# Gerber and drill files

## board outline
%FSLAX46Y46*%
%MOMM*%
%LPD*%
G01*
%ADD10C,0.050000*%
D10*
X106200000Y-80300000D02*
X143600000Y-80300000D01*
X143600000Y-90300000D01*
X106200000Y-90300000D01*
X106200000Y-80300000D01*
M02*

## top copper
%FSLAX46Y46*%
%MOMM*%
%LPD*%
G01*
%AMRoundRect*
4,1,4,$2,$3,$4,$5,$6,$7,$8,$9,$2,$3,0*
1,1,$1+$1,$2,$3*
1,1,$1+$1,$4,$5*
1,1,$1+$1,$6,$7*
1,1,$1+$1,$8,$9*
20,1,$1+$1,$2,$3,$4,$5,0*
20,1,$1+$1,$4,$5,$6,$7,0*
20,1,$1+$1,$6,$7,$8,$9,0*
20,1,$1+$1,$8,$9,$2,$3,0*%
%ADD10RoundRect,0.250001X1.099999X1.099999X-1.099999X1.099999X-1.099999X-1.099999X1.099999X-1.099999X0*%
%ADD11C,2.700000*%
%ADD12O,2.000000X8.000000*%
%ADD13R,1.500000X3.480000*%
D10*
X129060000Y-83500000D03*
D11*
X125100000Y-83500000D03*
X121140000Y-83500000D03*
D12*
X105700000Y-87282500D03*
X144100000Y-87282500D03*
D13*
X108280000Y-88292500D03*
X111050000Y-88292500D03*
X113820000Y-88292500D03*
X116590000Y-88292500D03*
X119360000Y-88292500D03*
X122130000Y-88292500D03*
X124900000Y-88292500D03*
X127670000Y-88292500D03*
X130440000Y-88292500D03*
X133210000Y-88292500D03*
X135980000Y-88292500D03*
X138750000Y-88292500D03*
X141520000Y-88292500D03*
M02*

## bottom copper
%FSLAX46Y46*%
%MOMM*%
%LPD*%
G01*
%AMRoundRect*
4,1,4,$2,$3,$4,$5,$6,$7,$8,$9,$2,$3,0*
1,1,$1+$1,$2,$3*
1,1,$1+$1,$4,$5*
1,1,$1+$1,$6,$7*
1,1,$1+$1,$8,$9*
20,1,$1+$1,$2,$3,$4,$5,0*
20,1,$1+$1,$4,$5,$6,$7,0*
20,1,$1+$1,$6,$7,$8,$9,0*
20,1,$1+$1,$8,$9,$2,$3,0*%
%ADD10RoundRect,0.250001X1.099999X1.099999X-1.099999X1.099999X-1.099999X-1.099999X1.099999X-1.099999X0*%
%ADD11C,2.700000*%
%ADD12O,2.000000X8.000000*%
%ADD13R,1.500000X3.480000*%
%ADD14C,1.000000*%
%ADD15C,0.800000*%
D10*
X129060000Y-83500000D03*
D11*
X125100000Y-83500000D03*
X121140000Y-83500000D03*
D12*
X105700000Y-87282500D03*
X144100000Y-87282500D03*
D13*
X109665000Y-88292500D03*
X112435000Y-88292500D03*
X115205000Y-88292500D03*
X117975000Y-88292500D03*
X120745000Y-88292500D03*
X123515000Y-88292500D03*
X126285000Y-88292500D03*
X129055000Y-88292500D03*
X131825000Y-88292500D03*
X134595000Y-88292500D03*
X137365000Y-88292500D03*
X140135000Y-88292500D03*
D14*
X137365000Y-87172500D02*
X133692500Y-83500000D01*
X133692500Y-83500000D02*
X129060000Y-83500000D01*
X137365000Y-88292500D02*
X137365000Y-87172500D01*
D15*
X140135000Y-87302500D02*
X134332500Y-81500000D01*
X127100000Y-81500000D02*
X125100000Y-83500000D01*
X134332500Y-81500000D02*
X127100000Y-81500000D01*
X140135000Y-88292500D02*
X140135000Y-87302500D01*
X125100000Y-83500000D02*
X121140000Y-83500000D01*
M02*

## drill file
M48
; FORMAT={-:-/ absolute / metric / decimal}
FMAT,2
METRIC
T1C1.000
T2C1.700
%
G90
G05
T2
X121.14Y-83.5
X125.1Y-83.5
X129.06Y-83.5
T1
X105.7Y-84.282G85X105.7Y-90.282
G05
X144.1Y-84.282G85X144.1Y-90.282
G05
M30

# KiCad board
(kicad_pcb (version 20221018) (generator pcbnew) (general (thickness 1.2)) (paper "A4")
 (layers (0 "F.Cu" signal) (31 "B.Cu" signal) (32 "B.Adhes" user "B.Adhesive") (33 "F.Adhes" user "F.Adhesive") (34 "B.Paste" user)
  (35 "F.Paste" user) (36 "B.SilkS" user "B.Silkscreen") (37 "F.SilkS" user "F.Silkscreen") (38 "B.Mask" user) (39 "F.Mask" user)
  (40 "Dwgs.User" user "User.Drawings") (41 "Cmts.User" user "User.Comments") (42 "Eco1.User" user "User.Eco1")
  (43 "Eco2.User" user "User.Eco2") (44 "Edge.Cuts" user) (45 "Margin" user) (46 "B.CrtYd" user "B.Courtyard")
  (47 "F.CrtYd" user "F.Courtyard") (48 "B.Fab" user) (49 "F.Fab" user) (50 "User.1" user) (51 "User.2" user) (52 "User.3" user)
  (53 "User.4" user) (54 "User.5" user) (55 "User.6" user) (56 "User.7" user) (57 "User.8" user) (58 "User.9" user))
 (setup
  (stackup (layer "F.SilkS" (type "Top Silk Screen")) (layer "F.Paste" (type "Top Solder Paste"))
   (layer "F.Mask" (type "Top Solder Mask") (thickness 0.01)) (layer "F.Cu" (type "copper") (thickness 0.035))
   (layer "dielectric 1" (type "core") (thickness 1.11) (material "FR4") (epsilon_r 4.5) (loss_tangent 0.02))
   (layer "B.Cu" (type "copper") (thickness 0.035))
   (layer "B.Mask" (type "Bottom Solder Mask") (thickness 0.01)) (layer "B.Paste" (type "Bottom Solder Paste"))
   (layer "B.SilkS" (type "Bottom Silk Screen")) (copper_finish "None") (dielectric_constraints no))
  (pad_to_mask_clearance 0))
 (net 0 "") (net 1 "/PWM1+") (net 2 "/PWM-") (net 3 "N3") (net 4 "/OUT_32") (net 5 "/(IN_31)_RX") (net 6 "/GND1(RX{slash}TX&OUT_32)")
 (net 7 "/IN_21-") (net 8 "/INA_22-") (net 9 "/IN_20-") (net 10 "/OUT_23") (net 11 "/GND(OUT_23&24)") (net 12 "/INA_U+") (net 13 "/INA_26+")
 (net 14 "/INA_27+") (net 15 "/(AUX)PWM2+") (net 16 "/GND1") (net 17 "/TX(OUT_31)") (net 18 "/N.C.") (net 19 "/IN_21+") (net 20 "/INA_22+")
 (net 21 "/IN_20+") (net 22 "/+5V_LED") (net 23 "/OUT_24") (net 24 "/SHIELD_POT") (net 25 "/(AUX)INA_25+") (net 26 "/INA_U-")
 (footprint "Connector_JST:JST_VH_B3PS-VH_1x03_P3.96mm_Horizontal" (layer "F.Cu") (at 129.06 83.5 180)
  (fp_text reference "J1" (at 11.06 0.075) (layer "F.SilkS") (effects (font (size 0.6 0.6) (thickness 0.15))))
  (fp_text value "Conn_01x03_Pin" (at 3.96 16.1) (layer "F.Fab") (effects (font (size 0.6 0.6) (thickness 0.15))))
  (pad "1" thru_hole roundrect (at 0 0 180) (size 2.7 2.7) (drill 1.7) (layers "*.Cu" "*.Mask") (roundrect_rratio 0.092593) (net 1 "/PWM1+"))
  (pad "2" thru_hole circle (at 3.96 0 180) (size 2.7 2.7) (drill 1.7) (layers "*.Cu" "*.Mask") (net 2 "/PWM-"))
  (pad "3" thru_hole circle (at 7.92 0 180) (size 2.7 2.7) (drill 1.7) (layers "*.Cu" "*.Mask") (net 2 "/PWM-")))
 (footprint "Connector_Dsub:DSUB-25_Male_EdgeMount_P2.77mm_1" (layer "F.Cu") (at 124.9 88.2925)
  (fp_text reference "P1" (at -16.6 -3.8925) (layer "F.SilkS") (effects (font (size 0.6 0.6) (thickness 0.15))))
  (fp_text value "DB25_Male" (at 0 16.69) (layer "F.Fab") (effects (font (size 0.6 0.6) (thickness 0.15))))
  (pad "0" thru_hole oval (at -19.2 -1.01) (size 2 8) (drill oval 1 7) (layers "*.Cu" "*.Mask") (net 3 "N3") (thermal_bridge_angle 45))
  (pad "0" thru_hole oval (at 19.2 -1.01) (size 2 8) (drill oval 1 7) (layers "*.Cu" "*.Mask") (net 3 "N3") (thermal_bridge_angle 45))
  (pad "1" smd rect (at -16.62 0) (size 1.5 3.48) (layers "F.Cu" "F.Paste" "F.Mask") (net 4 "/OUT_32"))
  (pad "2" smd rect (at -13.85 0) (size 1.5 3.48) (layers "F.Cu" "F.Paste" "F.Mask") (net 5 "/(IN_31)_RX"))
  (pad "3" smd rect (at -11.08 0) (size 1.5 3.48) (layers "F.Cu" "F.Paste" "F.Mask") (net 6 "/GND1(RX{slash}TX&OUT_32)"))
  (pad "4" smd rect (at -8.31 0) (size 1.5 3.48) (layers "F.Cu" "F.Paste" "F.Mask") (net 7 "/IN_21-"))
  (pad "5" smd rect (at -5.54 0) (size 1.5 3.48) (layers "F.Cu" "F.Paste" "F.Mask") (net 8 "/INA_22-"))
  (pad "6" smd rect (at -2.77 0) (size 1.5 3.48) (layers "F.Cu" "F.Paste" "F.Mask") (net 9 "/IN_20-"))
  (pad "7" smd rect (at 0 0) (size 1.5 3.48) (layers "F.Cu" "F.Paste" "F.Mask") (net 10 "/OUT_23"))
  (pad "8" smd rect (at 2.77 0) (size 1.5 3.48) (layers "F.Cu" "F.Paste" "F.Mask") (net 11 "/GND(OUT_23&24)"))
  (pad "9" smd rect (at 5.54 0) (size 1.5 3.48) (layers "F.Cu" "F.Paste" "F.Mask") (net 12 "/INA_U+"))
  (pad "10" smd rect (at 8.31 0) (size 1.5 3.48) (layers "F.Cu" "F.Paste" "F.Mask") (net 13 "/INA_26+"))
  (pad "11" smd rect (at 11.08 0) (size 1.5 3.48) (layers "F.Cu" "F.Paste" "F.Mask") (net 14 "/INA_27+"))
  (pad "12" smd rect (at 13.85 0) (size 1.5 3.48) (layers "F.Cu" "F.Paste" "F.Mask") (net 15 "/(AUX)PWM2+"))
  (pad "13" smd rect (at 16.62 0) (size 1.5 3.48) (layers "F.Cu" "F.Paste" "F.Mask") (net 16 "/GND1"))
  (pad "14" smd rect (at -15.235 0) (size 1.5 3.48) (layers "B.Cu" "B.Paste" "B.Mask") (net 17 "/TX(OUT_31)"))
  (pad "15" smd rect (at -12.465 0) (size 1.5 3.48) (layers "B.Cu" "B.Paste" "B.Mask") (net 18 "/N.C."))
  (pad "16" smd rect (at -9.695 0) (size 1.5 3.48) (layers "B.Cu" "B.Paste" "B.Mask") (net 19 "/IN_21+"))
  (pad "17" smd rect (at -6.925 0) (size 1.5 3.48) (layers "B.Cu" "B.Paste" "B.Mask") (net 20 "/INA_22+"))
  (pad "18" smd rect (at -4.155 0) (size 1.5 3.48) (layers "B.Cu" "B.Paste" "B.Mask") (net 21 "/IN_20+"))
  (pad "19" smd rect (at -1.385 0) (size 1.5 3.48) (layers "B.Cu" "B.Paste" "B.Mask") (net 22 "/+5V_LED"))
  (pad "20" smd rect (at 1.385 0) (size 1.5 3.48) (layers "B.Cu" "B.Paste" "B.Mask") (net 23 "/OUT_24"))
  (pad "21" smd rect (at 4.155 0) (size 1.5 3.48) (layers "B.Cu" "B.Paste" "B.Mask") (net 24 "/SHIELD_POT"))
  (pad "22" smd rect (at 6.925 0) (size 1.5 3.48) (layers "B.Cu" "B.Paste" "B.Mask") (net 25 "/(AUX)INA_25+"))
  (pad "23" smd rect (at 9.695 0) (size 1.5 3.48) (layers "B.Cu" "B.Paste" "B.Mask") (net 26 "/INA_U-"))
  (pad "24" smd rect (at 12.465 0) (size 1.5 3.48) (layers "B.Cu" "B.Paste" "B.Mask") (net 1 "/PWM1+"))
  (pad "25" smd rect (at 15.235 0) (size 1.5 3.48) (layers "B.Cu" "B.Paste" "B.Mask") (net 2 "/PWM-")))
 (gr_rect (start 106.2 80.3) (end 143.6 90.3) (stroke (width 0.05) (type default)) (fill none) (layer "Edge.Cuts"))
 (segment (start 137.365 87.1725) (end 133.6925 83.5) (width 1) (layer "B.Cu") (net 1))
 (segment (start 133.6925 83.5) (end 129.06 83.5) (width 1) (layer "B.Cu") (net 1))
 (segment (start 137.365 88.2925) (end 137.365 87.1725) (width 1) (layer "B.Cu") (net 1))
 (segment (start 140.135 87.3025) (end 134.3325 81.5) (width 0.8) (layer "B.Cu") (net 2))
 (segment (start 127.1 81.5) (end 125.1 83.5) (width 0.8) (layer "B.Cu") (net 2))
 (segment (start 134.3325 81.5) (end 127.1 81.5) (width 0.8) (layer "B.Cu") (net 2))
 (segment (start 140.135 88.2925) (end 140.135 87.3025) (width 0.8) (layer "B.Cu") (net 2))
 (segment (start 125.1 83.5) (end 121.14 83.5) (width 0.8) (layer "B.Cu") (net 2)))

